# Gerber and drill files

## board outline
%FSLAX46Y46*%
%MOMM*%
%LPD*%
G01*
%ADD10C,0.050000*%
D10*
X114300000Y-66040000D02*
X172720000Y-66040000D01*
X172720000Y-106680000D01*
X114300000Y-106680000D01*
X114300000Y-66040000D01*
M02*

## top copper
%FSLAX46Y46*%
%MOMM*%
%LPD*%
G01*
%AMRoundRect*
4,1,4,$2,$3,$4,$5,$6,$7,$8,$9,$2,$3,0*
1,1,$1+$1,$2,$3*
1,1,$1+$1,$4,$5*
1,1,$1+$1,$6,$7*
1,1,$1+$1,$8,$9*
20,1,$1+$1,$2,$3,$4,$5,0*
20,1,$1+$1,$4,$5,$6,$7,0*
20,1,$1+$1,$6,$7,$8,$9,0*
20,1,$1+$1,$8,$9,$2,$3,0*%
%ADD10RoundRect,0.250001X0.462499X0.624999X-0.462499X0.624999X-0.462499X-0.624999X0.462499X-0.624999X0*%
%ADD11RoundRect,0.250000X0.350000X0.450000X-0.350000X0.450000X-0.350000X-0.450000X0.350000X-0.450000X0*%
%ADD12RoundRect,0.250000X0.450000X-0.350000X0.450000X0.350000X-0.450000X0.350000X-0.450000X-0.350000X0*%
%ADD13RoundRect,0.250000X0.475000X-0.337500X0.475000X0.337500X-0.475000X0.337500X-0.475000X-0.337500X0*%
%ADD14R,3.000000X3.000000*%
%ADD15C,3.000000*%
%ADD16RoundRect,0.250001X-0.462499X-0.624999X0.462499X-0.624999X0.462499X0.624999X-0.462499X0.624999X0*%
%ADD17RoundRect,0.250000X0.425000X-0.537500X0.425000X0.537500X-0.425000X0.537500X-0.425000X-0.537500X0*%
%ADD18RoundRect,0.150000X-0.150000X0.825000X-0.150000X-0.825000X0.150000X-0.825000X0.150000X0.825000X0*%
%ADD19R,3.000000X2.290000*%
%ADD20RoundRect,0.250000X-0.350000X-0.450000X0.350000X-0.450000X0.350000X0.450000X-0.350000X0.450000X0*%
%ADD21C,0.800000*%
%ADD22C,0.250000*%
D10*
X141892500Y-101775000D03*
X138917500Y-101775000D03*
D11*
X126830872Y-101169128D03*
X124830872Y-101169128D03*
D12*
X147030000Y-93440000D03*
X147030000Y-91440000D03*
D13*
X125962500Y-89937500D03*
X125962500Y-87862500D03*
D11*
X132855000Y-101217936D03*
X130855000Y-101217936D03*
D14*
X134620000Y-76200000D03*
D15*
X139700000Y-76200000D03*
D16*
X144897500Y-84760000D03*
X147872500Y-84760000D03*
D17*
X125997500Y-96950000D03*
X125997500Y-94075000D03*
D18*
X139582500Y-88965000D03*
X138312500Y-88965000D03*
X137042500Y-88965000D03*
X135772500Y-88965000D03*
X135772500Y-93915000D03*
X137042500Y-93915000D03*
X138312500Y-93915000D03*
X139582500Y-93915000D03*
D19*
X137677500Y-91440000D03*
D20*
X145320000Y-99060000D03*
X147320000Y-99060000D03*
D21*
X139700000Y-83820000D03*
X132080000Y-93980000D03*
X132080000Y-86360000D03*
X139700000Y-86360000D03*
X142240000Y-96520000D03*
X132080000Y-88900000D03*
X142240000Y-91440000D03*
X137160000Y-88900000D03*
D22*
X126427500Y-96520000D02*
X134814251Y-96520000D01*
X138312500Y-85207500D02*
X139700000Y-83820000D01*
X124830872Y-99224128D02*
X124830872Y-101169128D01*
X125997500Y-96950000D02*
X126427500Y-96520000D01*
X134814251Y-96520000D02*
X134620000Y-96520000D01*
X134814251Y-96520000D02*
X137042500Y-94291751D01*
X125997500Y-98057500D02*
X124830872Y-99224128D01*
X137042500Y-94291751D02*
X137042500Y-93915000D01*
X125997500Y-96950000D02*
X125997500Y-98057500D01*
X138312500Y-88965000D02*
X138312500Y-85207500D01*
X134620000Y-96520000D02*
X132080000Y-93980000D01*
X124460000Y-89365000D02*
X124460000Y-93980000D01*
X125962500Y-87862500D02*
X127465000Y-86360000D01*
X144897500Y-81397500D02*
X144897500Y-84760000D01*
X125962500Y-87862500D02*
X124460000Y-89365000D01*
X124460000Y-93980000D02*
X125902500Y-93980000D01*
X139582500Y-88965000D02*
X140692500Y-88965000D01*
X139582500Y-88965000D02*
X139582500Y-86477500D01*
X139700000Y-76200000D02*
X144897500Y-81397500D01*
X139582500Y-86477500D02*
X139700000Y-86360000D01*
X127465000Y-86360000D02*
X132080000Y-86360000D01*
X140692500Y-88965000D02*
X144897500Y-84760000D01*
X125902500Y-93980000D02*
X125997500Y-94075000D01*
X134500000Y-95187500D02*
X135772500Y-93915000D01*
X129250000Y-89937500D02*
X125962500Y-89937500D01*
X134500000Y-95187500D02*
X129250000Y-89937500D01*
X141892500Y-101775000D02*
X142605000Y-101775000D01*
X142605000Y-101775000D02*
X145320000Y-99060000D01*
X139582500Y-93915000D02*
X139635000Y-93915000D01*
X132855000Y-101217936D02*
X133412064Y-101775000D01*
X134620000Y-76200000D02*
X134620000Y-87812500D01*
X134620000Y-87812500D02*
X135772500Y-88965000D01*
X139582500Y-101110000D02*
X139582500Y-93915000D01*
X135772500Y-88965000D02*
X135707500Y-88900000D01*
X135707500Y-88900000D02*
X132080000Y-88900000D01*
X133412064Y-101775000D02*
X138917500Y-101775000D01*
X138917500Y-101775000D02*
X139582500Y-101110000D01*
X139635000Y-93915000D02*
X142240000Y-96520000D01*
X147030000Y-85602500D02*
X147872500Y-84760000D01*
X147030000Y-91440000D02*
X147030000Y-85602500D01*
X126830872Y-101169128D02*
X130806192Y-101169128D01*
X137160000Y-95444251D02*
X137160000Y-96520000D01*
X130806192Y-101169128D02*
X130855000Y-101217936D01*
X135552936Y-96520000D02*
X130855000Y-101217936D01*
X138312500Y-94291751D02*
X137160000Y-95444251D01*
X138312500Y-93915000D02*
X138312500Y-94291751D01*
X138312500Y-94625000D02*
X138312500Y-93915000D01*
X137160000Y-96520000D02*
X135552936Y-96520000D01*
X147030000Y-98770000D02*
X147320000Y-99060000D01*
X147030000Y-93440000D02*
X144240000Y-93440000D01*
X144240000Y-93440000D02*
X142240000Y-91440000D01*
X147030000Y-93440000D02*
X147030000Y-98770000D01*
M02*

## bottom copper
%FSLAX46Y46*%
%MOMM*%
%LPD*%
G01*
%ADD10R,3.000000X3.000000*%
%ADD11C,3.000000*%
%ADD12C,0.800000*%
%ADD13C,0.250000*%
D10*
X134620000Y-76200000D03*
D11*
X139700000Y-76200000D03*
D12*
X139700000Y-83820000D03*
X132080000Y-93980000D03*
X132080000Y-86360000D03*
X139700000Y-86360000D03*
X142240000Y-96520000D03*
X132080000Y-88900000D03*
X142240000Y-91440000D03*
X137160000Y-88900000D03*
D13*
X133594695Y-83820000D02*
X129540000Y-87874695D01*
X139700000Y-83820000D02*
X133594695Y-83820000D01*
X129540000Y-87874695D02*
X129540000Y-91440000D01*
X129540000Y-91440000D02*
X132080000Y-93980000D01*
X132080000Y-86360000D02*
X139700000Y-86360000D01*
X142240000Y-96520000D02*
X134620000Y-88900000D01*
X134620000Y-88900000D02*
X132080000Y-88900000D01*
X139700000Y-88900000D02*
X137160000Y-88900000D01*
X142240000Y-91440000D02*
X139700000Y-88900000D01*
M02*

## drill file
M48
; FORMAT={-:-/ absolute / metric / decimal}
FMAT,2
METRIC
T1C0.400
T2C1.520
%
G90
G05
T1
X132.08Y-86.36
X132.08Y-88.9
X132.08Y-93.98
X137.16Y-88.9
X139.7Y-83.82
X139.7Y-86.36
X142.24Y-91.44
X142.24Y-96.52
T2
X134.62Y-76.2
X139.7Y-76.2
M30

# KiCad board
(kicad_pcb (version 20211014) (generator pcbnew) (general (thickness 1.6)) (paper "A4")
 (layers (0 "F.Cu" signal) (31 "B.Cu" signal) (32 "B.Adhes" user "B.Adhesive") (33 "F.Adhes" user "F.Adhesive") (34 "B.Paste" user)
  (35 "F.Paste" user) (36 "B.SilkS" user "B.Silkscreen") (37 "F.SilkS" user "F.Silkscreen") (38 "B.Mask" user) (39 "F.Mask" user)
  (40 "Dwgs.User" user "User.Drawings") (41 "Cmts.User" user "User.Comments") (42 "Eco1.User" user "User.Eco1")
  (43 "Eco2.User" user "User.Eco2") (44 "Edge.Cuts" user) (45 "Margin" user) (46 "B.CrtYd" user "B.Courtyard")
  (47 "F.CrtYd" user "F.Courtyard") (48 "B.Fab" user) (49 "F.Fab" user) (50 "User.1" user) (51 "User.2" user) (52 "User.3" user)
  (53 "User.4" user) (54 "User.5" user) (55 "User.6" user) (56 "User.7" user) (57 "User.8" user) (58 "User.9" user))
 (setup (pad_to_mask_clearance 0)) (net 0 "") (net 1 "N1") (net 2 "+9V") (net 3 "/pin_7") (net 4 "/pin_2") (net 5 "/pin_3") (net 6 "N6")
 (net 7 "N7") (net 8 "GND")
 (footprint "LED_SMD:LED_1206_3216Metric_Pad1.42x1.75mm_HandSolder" (layer "F.Cu") (at 140.405 101.775 180)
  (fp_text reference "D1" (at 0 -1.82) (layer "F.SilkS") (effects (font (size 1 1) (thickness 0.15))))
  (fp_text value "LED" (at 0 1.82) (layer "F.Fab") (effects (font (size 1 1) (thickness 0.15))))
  (pad "1" smd roundrect (at -1.4875 0 180) (size 1.425 1.75) (layers "F.Cu" "F.Paste" "F.Mask") (roundrect_rratio 0.175439) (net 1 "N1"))
  (pad "2" smd roundrect (at 1.4875 0 180) (size 1.425 1.75) (layers "F.Cu" "F.Paste" "F.Mask") (roundrect_rratio 0.175439) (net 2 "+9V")))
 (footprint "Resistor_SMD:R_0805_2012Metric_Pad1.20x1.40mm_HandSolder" (layer "F.Cu") (at 125.830872 101.169128 180)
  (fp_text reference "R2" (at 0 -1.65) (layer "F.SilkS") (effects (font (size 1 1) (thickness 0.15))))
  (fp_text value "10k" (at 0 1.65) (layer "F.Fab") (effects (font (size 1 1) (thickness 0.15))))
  (pad "1" smd roundrect (at -1 0 180) (size 1.2 1.4) (layers "F.Cu" "F.Paste" "F.Mask") (roundrect_rratio 0.208333) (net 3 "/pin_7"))
  (pad "2" smd roundrect (at 1 0 180) (size 1.2 1.4) (layers "F.Cu" "F.Paste" "F.Mask") (roundrect_rratio 0.208333) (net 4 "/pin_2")))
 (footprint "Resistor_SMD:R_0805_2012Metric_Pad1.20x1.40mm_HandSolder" (layer "F.Cu") (at 147.03 92.44 90)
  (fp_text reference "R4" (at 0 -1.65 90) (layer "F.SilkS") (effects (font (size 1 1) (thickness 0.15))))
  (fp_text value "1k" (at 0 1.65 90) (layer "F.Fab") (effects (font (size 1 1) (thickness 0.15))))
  (pad "1" smd roundrect (at -1 0 90) (size 1.2 1.4) (layers "F.Cu" "F.Paste" "F.Mask") (roundrect_rratio 0.208333) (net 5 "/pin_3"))
  (pad "2" smd roundrect (at 1 0 90) (size 1.2 1.4) (layers "F.Cu" "F.Paste" "F.Mask") (roundrect_rratio 0.208333) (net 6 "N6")))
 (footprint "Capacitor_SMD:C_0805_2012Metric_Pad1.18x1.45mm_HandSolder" (layer "F.Cu") (at 125.9625 88.9 90)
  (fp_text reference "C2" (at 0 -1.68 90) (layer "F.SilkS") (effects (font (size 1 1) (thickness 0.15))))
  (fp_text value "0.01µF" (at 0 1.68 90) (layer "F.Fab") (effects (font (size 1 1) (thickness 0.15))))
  (pad "1" smd roundrect (at -1.0375 0 90) (size 1.175 1.45) (layers "F.Cu" "F.Paste" "F.Mask") (roundrect_rratio 0.212766) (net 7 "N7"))
  (pad "2" smd roundrect (at 1.0375 0 90) (size 1.175 1.45) (layers "F.Cu" "F.Paste" "F.Mask") (roundrect_rratio 0.212766) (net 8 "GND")))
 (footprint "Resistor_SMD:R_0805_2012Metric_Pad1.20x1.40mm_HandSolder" (layer "F.Cu") (at 131.855 101.217936 180)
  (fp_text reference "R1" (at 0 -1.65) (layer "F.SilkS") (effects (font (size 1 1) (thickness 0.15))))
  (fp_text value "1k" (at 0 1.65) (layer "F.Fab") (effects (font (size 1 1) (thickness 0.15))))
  (pad "1" smd roundrect (at -1 0 180) (size 1.2 1.4) (layers "F.Cu" "F.Paste" "F.Mask") (roundrect_rratio 0.208333) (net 2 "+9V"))
  (pad "2" smd roundrect (at 1 0 180) (size 1.2 1.4) (layers "F.Cu" "F.Paste" "F.Mask") (roundrect_rratio 0.208333) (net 3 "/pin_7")))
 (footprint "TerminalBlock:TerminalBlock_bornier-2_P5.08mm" (layer "F.Cu") (at 134.62 76.2)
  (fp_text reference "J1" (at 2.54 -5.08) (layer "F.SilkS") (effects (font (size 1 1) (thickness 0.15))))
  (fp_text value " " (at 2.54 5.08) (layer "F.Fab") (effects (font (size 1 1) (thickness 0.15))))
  (pad "1" thru_hole rect (at 0 0) (size 3 3) (drill 1.52) (layers *.Cu *.Mask) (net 2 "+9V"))
  (pad "2" thru_hole circle (at 5.08 0) (size 3 3) (drill 1.52) (layers *.Cu *.Mask) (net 8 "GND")))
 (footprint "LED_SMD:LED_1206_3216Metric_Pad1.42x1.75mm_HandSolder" (layer "F.Cu") (at 146.385 84.76)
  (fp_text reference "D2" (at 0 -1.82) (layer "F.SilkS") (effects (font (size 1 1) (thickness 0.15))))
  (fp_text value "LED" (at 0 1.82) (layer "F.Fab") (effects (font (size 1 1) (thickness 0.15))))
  (pad "1" smd roundrect (at -1.4875 0) (size 1.425 1.75) (layers "F.Cu" "F.Paste" "F.Mask") (roundrect_rratio 0.175439) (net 8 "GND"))
  (pad "2" smd roundrect (at 1.4875 0) (size 1.425 1.75) (layers "F.Cu" "F.Paste" "F.Mask") (roundrect_rratio 0.175439) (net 6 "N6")))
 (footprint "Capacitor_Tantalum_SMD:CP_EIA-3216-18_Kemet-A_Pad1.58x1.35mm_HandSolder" (layer "F.Cu") (at 125.9975 95.5125 90)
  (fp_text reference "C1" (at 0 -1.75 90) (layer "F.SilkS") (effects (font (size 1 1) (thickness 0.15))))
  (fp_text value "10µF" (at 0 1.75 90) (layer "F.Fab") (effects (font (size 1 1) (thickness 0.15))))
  (pad "1" smd roundrect (at -1.4375 0 90) (size 1.575 1.35) (layers "F.Cu" "F.Paste" "F.Mask") (roundrect_rratio 0.185185) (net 4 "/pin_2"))
  (pad "2" smd roundrect (at 1.4375 0 90) (size 1.575 1.35) (layers "F.Cu" "F.Paste" "F.Mask") (roundrect_rratio 0.185185) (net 8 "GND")))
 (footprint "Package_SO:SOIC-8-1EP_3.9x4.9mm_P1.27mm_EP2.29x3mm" (layer "F.Cu") (at 137.6775 91.44 -90)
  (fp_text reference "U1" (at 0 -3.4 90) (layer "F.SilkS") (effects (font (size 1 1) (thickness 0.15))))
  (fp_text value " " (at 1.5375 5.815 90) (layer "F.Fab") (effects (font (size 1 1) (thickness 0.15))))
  (pad "" smd roundrect (at -0.57 -0.75 270) (size 0.92 1.21) (layers "F.Paste") (roundrect_rratio 0.25))
  (pad "" smd roundrect (at 0.57 -0.75 270) (size 0.92 1.21) (layers "F.Paste") (roundrect_rratio 0.25))
  (pad "" smd roundrect (at -0.57 0.75 270) (size 0.92 1.21) (layers "F.Paste") (roundrect_rratio 0.25))
  (pad "" smd roundrect (at 0.57 0.75 270) (size 0.92 1.21) (layers "F.Paste") (roundrect_rratio 0.25))
  (pad "1" smd roundrect (at -2.475 -1.905 270) (size 1.95 0.6) (layers "F.Cu" "F.Paste" "F.Mask") (roundrect_rratio 0.25) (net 8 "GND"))
  (pad "2" smd roundrect (at -2.475 -0.635 270) (size 1.95 0.6) (layers "F.Cu" "F.Paste" "F.Mask") (roundrect_rratio 0.25) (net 4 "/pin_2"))
  (pad "3" smd roundrect (at -2.475 0.635 270) (size 1.95 0.6) (layers "F.Cu" "F.Paste" "F.Mask") (roundrect_rratio 0.25) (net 5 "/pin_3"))
  (pad "4" smd roundrect (at -2.475 1.905 270) (size 1.95 0.6) (layers "F.Cu" "F.Paste" "F.Mask") (roundrect_rratio 0.25) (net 2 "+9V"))
  (pad "5" smd roundrect (at 2.475 1.905 270) (size 1.95 0.6) (layers "F.Cu" "F.Paste" "F.Mask") (roundrect_rratio 0.25) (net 7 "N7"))
  (pad "6" smd roundrect (at 2.475 0.635 270) (size 1.95 0.6) (layers "F.Cu" "F.Paste" "F.Mask") (roundrect_rratio 0.25) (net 4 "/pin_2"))
  (pad "7" smd roundrect (at 2.475 -0.635 270) (size 1.95 0.6) (layers "F.Cu" "F.Paste" "F.Mask") (roundrect_rratio 0.25) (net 3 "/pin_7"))
  (pad "8" smd roundrect (at 2.475 -1.905 270) (size 1.95 0.6) (layers "F.Cu" "F.Paste" "F.Mask") (roundrect_rratio 0.25) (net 2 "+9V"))
  (pad "9" smd rect (at 0 0 270) (size 2.29 3) (layers "F.Cu" "F.Mask")))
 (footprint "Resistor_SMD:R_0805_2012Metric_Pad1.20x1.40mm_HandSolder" (layer "F.Cu") (at 146.32 99.06)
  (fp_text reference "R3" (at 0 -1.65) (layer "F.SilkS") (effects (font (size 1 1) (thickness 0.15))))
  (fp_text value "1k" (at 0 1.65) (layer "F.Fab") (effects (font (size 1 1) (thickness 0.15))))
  (pad "1" smd roundrect (at -1 0) (size 1.2 1.4) (layers "F.Cu" "F.Paste" "F.Mask") (roundrect_rratio 0.208333) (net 1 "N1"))
  (pad "2" smd roundrect (at 1 0) (size 1.2 1.4) (layers "F.Cu" "F.Paste" "F.Mask") (roundrect_rratio 0.208333) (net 5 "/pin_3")))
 (gr_rect (start 114.3 66.04) (end 172.72 106.68) (layer "Edge.Cuts") (width 0.05) (fill none))
 (segment (start 126.4275 96.52) (end 134.814251 96.52) (width 0.25) (layer "F.Cu") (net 4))
 (segment (start 138.3125 85.2075) (end 139.7 83.82) (width 0.25) (layer "F.Cu") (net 4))
 (segment (start 124.830872 99.224128) (end 124.830872 101.169128) (width 0.25) (layer "F.Cu") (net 4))
 (segment (start 125.9975 96.95) (end 126.4275 96.52) (width 0.25) (layer "F.Cu") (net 4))
 (segment (start 134.814251 96.52) (end 134.62 96.52) (width 0.25) (layer "F.Cu") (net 4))
 (segment (start 134.814251 96.52) (end 137.0425 94.291751) (width 0.25) (layer "F.Cu") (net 4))
 (segment (start 125.9975 98.0575) (end 124.830872 99.224128) (width 0.25) (layer "F.Cu") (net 4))
 (segment (start 137.0425 94.291751) (end 137.0425 93.915) (width 0.25) (layer "F.Cu") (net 4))
 (segment (start 125.9975 96.95) (end 125.9975 98.0575) (width 0.25) (layer "F.Cu") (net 4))
 (segment (start 138.3125 88.965) (end 138.3125 85.2075) (width 0.25) (layer "F.Cu") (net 4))
 (segment (start 134.62 96.52) (end 132.08 93.98) (width 0.25) (layer "F.Cu") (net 4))
 (via (at 139.7 83.82) (size 0.8) (drill 0.4) (layers "F.Cu" "B.Cu") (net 4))
 (via (at 132.08 93.98) (size 0.8) (drill 0.4) (layers "F.Cu" "B.Cu") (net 4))
 (segment (start 133.594695 83.82) (end 129.54 87.874695) (width 0.25) (layer "B.Cu") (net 4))
 (segment (start 139.7 83.82) (end 133.594695 83.82) (width 0.25) (layer "B.Cu") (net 4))
 (segment (start 129.54 87.874695) (end 129.54 91.44) (width 0.25) (layer "B.Cu") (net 4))
 (segment (start 129.54 91.44) (end 132.08 93.98) (width 0.25) (layer "B.Cu") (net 4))
 (segment (start 124.46 89.365) (end 124.46 93.98) (width 0.25) (layer "F.Cu") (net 8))
 (segment (start 125.9625 87.8625) (end 127.465 86.36) (width 0.25) (layer "F.Cu") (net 8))
 (segment (start 144.8975 81.3975) (end 144.8975 84.76) (width 0.25) (layer "F.Cu") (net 8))
 (segment (start 125.9625 87.8625) (end 124.46 89.365) (width 0.25) (layer "F.Cu") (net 8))
 (segment (start 124.46 93.98) (end 125.9025 93.98) (width 0.25) (layer "F.Cu") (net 8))
 (segment (start 139.5825 88.965) (end 140.6925 88.965) (width 0.25) (layer "F.Cu") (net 8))
 (segment (start 139.5825 88.965) (end 139.5825 86.4775) (width 0.25) (layer "F.Cu") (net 8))
 (segment (start 139.7 76.2) (end 144.8975 81.3975) (width 0.25) (layer "F.Cu") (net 8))
 (segment (start 139.5825 86.4775) (end 139.7 86.36) (width 0.25) (layer "F.Cu") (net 8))
 (segment (start 127.465 86.36) (end 132.08 86.36) (width 0.25) (layer "F.Cu") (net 8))
 (segment (start 140.6925 88.965) (end 144.8975 84.76) (width 0.25) (layer "F.Cu") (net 8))
 (segment (start 125.9025 93.98) (end 125.9975 94.075) (width 0.25) (layer "F.Cu") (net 8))
 (via (at 132.08 86.36) (size 0.8) (drill 0.4) (layers "F.Cu" "B.Cu") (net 8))
 (via (at 139.7 86.36) (size 0.8) (drill 0.4) (layers "F.Cu" "B.Cu") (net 8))
 (segment (start 132.08 86.36) (end 139.7 86.36) (width 0.25) (layer "B.Cu") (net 8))
 (segment (start 134.5 95.1875) (end 135.7725 93.915) (width 0.25) (layer "F.Cu") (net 7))
 (segment (start 129.25 89.9375) (end 125.9625 89.9375) (width 0.25) (layer "F.Cu") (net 7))
 (segment (start 134.5 95.1875) (end 129.25 89.9375) (width 0.25) (layer "F.Cu") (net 7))
 (segment (start 141.8925 101.775) (end 142.605 101.775) (width 0.25) (layer "F.Cu") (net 1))
 (segment (start 142.605 101.775) (end 145.32 99.06) (width 0.25) (layer "F.Cu") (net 1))
 (segment (start 139.5825 93.915) (end 139.635 93.915) (width 0.25) (layer "F.Cu") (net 2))
 (segment (start 132.855 101.217936) (end 133.412064 101.775) (width 0.25) (layer "F.Cu") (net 2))
 (segment (start 134.62 76.2) (end 134.62 87.8125) (width 0.25) (layer "F.Cu") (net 2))
 (segment (start 134.62 87.8125) (end 135.7725 88.965) (width 0.25) (layer "F.Cu") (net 2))
 (segment (start 139.5825 101.11) (end 139.5825 93.915) (width 0.25) (layer "F.Cu") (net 2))
 (segment (start 135.7725 88.965) (end 135.7075 88.9) (width 0.25) (layer "F.Cu") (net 2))
 (segment (start 135.7075 88.9) (end 132.08 88.9) (width 0.25) (layer "F.Cu") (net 2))
 (segment (start 133.412064 101.775) (end 138.9175 101.775) (width 0.25) (layer "F.Cu") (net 2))
 (segment (start 138.9175 101.775) (end 139.5825 101.11) (width 0.25) (layer "F.Cu") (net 2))
 (segment (start 139.635 93.915) (end 142.24 96.52) (width 0.25) (layer "F.Cu") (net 2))
 (via (at 142.24 96.52) (size 0.8) (drill 0.4) (layers "F.Cu" "B.Cu") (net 2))
 (via (at 132.08 88.9) (size 0.8) (drill 0.4) (layers "F.Cu" "B.Cu") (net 2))
 (segment (start 142.24 96.52) (end 134.62 88.9) (width 0.25) (layer "B.Cu") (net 2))
 (segment (start 134.62 88.9) (end 132.08 88.9) (width 0.25) (layer "B.Cu") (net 2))
 (segment (start 147.03 85.6025) (end 147.8725 84.76) (width 0.25) (layer "F.Cu") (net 6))
 (segment (start 147.03 91.44) (end 147.03 85.6025) (width 0.25) (layer "F.Cu") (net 6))
 (segment (start 126.830872 101.169128) (end 130.806192 101.169128) (width 0.25) (layer "F.Cu") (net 3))
 (segment (start 137.16 95.444251) (end 137.16 96.52) (width 0.25) (layer "F.Cu") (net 3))
 (segment (start 130.806192 101.169128) (end 130.855 101.217936) (width 0.25) (layer "F.Cu") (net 3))
 (segment (start 135.552936 96.52) (end 130.855 101.217936) (width 0.25) (layer "F.Cu") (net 3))
 (segment (start 138.3125 94.291751) (end 137.16 95.444251) (width 0.25) (layer "F.Cu") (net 3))
 (segment (start 138.3125 93.915) (end 138.3125 94.291751) (width 0.25) (layer "F.Cu") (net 3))
 (segment (start 138.3125 94.625) (end 138.3125 93.915) (width 0.25) (layer "F.Cu") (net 3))
 (segment (start 137.16 96.52) (end 135.552936 96.52) (width 0.25) (layer "F.Cu") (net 3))
 (segment (start 147.03 98.77) (end 147.32 99.06) (width 0.25) (layer "F.Cu") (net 5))
 (segment (start 147.03 93.44) (end 144.24 93.44) (width 0.25) (layer "F.Cu") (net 5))
 (segment (start 144.24 93.44) (end 142.24 91.44) (width 0.25) (layer "F.Cu") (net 5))
 (segment (start 147.03 93.44) (end 147.03 98.77) (width 0.25) (layer "F.Cu") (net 5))
 (via (at 142.24 91.44) (size 0.8) (drill 0.4) (layers "F.Cu" "B.Cu") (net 5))
 (via (at 137.16 88.9) (size 0.8) (drill 0.4) (layers "F.Cu" "B.Cu") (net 5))
 (segment (start 139.7 88.9) (end 137.16 88.9) (width 0.25) (layer "B.Cu") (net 5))
 (segment (start 142.24 91.44) (end 139.7 88.9) (width 0.25) (layer "B.Cu") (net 5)))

